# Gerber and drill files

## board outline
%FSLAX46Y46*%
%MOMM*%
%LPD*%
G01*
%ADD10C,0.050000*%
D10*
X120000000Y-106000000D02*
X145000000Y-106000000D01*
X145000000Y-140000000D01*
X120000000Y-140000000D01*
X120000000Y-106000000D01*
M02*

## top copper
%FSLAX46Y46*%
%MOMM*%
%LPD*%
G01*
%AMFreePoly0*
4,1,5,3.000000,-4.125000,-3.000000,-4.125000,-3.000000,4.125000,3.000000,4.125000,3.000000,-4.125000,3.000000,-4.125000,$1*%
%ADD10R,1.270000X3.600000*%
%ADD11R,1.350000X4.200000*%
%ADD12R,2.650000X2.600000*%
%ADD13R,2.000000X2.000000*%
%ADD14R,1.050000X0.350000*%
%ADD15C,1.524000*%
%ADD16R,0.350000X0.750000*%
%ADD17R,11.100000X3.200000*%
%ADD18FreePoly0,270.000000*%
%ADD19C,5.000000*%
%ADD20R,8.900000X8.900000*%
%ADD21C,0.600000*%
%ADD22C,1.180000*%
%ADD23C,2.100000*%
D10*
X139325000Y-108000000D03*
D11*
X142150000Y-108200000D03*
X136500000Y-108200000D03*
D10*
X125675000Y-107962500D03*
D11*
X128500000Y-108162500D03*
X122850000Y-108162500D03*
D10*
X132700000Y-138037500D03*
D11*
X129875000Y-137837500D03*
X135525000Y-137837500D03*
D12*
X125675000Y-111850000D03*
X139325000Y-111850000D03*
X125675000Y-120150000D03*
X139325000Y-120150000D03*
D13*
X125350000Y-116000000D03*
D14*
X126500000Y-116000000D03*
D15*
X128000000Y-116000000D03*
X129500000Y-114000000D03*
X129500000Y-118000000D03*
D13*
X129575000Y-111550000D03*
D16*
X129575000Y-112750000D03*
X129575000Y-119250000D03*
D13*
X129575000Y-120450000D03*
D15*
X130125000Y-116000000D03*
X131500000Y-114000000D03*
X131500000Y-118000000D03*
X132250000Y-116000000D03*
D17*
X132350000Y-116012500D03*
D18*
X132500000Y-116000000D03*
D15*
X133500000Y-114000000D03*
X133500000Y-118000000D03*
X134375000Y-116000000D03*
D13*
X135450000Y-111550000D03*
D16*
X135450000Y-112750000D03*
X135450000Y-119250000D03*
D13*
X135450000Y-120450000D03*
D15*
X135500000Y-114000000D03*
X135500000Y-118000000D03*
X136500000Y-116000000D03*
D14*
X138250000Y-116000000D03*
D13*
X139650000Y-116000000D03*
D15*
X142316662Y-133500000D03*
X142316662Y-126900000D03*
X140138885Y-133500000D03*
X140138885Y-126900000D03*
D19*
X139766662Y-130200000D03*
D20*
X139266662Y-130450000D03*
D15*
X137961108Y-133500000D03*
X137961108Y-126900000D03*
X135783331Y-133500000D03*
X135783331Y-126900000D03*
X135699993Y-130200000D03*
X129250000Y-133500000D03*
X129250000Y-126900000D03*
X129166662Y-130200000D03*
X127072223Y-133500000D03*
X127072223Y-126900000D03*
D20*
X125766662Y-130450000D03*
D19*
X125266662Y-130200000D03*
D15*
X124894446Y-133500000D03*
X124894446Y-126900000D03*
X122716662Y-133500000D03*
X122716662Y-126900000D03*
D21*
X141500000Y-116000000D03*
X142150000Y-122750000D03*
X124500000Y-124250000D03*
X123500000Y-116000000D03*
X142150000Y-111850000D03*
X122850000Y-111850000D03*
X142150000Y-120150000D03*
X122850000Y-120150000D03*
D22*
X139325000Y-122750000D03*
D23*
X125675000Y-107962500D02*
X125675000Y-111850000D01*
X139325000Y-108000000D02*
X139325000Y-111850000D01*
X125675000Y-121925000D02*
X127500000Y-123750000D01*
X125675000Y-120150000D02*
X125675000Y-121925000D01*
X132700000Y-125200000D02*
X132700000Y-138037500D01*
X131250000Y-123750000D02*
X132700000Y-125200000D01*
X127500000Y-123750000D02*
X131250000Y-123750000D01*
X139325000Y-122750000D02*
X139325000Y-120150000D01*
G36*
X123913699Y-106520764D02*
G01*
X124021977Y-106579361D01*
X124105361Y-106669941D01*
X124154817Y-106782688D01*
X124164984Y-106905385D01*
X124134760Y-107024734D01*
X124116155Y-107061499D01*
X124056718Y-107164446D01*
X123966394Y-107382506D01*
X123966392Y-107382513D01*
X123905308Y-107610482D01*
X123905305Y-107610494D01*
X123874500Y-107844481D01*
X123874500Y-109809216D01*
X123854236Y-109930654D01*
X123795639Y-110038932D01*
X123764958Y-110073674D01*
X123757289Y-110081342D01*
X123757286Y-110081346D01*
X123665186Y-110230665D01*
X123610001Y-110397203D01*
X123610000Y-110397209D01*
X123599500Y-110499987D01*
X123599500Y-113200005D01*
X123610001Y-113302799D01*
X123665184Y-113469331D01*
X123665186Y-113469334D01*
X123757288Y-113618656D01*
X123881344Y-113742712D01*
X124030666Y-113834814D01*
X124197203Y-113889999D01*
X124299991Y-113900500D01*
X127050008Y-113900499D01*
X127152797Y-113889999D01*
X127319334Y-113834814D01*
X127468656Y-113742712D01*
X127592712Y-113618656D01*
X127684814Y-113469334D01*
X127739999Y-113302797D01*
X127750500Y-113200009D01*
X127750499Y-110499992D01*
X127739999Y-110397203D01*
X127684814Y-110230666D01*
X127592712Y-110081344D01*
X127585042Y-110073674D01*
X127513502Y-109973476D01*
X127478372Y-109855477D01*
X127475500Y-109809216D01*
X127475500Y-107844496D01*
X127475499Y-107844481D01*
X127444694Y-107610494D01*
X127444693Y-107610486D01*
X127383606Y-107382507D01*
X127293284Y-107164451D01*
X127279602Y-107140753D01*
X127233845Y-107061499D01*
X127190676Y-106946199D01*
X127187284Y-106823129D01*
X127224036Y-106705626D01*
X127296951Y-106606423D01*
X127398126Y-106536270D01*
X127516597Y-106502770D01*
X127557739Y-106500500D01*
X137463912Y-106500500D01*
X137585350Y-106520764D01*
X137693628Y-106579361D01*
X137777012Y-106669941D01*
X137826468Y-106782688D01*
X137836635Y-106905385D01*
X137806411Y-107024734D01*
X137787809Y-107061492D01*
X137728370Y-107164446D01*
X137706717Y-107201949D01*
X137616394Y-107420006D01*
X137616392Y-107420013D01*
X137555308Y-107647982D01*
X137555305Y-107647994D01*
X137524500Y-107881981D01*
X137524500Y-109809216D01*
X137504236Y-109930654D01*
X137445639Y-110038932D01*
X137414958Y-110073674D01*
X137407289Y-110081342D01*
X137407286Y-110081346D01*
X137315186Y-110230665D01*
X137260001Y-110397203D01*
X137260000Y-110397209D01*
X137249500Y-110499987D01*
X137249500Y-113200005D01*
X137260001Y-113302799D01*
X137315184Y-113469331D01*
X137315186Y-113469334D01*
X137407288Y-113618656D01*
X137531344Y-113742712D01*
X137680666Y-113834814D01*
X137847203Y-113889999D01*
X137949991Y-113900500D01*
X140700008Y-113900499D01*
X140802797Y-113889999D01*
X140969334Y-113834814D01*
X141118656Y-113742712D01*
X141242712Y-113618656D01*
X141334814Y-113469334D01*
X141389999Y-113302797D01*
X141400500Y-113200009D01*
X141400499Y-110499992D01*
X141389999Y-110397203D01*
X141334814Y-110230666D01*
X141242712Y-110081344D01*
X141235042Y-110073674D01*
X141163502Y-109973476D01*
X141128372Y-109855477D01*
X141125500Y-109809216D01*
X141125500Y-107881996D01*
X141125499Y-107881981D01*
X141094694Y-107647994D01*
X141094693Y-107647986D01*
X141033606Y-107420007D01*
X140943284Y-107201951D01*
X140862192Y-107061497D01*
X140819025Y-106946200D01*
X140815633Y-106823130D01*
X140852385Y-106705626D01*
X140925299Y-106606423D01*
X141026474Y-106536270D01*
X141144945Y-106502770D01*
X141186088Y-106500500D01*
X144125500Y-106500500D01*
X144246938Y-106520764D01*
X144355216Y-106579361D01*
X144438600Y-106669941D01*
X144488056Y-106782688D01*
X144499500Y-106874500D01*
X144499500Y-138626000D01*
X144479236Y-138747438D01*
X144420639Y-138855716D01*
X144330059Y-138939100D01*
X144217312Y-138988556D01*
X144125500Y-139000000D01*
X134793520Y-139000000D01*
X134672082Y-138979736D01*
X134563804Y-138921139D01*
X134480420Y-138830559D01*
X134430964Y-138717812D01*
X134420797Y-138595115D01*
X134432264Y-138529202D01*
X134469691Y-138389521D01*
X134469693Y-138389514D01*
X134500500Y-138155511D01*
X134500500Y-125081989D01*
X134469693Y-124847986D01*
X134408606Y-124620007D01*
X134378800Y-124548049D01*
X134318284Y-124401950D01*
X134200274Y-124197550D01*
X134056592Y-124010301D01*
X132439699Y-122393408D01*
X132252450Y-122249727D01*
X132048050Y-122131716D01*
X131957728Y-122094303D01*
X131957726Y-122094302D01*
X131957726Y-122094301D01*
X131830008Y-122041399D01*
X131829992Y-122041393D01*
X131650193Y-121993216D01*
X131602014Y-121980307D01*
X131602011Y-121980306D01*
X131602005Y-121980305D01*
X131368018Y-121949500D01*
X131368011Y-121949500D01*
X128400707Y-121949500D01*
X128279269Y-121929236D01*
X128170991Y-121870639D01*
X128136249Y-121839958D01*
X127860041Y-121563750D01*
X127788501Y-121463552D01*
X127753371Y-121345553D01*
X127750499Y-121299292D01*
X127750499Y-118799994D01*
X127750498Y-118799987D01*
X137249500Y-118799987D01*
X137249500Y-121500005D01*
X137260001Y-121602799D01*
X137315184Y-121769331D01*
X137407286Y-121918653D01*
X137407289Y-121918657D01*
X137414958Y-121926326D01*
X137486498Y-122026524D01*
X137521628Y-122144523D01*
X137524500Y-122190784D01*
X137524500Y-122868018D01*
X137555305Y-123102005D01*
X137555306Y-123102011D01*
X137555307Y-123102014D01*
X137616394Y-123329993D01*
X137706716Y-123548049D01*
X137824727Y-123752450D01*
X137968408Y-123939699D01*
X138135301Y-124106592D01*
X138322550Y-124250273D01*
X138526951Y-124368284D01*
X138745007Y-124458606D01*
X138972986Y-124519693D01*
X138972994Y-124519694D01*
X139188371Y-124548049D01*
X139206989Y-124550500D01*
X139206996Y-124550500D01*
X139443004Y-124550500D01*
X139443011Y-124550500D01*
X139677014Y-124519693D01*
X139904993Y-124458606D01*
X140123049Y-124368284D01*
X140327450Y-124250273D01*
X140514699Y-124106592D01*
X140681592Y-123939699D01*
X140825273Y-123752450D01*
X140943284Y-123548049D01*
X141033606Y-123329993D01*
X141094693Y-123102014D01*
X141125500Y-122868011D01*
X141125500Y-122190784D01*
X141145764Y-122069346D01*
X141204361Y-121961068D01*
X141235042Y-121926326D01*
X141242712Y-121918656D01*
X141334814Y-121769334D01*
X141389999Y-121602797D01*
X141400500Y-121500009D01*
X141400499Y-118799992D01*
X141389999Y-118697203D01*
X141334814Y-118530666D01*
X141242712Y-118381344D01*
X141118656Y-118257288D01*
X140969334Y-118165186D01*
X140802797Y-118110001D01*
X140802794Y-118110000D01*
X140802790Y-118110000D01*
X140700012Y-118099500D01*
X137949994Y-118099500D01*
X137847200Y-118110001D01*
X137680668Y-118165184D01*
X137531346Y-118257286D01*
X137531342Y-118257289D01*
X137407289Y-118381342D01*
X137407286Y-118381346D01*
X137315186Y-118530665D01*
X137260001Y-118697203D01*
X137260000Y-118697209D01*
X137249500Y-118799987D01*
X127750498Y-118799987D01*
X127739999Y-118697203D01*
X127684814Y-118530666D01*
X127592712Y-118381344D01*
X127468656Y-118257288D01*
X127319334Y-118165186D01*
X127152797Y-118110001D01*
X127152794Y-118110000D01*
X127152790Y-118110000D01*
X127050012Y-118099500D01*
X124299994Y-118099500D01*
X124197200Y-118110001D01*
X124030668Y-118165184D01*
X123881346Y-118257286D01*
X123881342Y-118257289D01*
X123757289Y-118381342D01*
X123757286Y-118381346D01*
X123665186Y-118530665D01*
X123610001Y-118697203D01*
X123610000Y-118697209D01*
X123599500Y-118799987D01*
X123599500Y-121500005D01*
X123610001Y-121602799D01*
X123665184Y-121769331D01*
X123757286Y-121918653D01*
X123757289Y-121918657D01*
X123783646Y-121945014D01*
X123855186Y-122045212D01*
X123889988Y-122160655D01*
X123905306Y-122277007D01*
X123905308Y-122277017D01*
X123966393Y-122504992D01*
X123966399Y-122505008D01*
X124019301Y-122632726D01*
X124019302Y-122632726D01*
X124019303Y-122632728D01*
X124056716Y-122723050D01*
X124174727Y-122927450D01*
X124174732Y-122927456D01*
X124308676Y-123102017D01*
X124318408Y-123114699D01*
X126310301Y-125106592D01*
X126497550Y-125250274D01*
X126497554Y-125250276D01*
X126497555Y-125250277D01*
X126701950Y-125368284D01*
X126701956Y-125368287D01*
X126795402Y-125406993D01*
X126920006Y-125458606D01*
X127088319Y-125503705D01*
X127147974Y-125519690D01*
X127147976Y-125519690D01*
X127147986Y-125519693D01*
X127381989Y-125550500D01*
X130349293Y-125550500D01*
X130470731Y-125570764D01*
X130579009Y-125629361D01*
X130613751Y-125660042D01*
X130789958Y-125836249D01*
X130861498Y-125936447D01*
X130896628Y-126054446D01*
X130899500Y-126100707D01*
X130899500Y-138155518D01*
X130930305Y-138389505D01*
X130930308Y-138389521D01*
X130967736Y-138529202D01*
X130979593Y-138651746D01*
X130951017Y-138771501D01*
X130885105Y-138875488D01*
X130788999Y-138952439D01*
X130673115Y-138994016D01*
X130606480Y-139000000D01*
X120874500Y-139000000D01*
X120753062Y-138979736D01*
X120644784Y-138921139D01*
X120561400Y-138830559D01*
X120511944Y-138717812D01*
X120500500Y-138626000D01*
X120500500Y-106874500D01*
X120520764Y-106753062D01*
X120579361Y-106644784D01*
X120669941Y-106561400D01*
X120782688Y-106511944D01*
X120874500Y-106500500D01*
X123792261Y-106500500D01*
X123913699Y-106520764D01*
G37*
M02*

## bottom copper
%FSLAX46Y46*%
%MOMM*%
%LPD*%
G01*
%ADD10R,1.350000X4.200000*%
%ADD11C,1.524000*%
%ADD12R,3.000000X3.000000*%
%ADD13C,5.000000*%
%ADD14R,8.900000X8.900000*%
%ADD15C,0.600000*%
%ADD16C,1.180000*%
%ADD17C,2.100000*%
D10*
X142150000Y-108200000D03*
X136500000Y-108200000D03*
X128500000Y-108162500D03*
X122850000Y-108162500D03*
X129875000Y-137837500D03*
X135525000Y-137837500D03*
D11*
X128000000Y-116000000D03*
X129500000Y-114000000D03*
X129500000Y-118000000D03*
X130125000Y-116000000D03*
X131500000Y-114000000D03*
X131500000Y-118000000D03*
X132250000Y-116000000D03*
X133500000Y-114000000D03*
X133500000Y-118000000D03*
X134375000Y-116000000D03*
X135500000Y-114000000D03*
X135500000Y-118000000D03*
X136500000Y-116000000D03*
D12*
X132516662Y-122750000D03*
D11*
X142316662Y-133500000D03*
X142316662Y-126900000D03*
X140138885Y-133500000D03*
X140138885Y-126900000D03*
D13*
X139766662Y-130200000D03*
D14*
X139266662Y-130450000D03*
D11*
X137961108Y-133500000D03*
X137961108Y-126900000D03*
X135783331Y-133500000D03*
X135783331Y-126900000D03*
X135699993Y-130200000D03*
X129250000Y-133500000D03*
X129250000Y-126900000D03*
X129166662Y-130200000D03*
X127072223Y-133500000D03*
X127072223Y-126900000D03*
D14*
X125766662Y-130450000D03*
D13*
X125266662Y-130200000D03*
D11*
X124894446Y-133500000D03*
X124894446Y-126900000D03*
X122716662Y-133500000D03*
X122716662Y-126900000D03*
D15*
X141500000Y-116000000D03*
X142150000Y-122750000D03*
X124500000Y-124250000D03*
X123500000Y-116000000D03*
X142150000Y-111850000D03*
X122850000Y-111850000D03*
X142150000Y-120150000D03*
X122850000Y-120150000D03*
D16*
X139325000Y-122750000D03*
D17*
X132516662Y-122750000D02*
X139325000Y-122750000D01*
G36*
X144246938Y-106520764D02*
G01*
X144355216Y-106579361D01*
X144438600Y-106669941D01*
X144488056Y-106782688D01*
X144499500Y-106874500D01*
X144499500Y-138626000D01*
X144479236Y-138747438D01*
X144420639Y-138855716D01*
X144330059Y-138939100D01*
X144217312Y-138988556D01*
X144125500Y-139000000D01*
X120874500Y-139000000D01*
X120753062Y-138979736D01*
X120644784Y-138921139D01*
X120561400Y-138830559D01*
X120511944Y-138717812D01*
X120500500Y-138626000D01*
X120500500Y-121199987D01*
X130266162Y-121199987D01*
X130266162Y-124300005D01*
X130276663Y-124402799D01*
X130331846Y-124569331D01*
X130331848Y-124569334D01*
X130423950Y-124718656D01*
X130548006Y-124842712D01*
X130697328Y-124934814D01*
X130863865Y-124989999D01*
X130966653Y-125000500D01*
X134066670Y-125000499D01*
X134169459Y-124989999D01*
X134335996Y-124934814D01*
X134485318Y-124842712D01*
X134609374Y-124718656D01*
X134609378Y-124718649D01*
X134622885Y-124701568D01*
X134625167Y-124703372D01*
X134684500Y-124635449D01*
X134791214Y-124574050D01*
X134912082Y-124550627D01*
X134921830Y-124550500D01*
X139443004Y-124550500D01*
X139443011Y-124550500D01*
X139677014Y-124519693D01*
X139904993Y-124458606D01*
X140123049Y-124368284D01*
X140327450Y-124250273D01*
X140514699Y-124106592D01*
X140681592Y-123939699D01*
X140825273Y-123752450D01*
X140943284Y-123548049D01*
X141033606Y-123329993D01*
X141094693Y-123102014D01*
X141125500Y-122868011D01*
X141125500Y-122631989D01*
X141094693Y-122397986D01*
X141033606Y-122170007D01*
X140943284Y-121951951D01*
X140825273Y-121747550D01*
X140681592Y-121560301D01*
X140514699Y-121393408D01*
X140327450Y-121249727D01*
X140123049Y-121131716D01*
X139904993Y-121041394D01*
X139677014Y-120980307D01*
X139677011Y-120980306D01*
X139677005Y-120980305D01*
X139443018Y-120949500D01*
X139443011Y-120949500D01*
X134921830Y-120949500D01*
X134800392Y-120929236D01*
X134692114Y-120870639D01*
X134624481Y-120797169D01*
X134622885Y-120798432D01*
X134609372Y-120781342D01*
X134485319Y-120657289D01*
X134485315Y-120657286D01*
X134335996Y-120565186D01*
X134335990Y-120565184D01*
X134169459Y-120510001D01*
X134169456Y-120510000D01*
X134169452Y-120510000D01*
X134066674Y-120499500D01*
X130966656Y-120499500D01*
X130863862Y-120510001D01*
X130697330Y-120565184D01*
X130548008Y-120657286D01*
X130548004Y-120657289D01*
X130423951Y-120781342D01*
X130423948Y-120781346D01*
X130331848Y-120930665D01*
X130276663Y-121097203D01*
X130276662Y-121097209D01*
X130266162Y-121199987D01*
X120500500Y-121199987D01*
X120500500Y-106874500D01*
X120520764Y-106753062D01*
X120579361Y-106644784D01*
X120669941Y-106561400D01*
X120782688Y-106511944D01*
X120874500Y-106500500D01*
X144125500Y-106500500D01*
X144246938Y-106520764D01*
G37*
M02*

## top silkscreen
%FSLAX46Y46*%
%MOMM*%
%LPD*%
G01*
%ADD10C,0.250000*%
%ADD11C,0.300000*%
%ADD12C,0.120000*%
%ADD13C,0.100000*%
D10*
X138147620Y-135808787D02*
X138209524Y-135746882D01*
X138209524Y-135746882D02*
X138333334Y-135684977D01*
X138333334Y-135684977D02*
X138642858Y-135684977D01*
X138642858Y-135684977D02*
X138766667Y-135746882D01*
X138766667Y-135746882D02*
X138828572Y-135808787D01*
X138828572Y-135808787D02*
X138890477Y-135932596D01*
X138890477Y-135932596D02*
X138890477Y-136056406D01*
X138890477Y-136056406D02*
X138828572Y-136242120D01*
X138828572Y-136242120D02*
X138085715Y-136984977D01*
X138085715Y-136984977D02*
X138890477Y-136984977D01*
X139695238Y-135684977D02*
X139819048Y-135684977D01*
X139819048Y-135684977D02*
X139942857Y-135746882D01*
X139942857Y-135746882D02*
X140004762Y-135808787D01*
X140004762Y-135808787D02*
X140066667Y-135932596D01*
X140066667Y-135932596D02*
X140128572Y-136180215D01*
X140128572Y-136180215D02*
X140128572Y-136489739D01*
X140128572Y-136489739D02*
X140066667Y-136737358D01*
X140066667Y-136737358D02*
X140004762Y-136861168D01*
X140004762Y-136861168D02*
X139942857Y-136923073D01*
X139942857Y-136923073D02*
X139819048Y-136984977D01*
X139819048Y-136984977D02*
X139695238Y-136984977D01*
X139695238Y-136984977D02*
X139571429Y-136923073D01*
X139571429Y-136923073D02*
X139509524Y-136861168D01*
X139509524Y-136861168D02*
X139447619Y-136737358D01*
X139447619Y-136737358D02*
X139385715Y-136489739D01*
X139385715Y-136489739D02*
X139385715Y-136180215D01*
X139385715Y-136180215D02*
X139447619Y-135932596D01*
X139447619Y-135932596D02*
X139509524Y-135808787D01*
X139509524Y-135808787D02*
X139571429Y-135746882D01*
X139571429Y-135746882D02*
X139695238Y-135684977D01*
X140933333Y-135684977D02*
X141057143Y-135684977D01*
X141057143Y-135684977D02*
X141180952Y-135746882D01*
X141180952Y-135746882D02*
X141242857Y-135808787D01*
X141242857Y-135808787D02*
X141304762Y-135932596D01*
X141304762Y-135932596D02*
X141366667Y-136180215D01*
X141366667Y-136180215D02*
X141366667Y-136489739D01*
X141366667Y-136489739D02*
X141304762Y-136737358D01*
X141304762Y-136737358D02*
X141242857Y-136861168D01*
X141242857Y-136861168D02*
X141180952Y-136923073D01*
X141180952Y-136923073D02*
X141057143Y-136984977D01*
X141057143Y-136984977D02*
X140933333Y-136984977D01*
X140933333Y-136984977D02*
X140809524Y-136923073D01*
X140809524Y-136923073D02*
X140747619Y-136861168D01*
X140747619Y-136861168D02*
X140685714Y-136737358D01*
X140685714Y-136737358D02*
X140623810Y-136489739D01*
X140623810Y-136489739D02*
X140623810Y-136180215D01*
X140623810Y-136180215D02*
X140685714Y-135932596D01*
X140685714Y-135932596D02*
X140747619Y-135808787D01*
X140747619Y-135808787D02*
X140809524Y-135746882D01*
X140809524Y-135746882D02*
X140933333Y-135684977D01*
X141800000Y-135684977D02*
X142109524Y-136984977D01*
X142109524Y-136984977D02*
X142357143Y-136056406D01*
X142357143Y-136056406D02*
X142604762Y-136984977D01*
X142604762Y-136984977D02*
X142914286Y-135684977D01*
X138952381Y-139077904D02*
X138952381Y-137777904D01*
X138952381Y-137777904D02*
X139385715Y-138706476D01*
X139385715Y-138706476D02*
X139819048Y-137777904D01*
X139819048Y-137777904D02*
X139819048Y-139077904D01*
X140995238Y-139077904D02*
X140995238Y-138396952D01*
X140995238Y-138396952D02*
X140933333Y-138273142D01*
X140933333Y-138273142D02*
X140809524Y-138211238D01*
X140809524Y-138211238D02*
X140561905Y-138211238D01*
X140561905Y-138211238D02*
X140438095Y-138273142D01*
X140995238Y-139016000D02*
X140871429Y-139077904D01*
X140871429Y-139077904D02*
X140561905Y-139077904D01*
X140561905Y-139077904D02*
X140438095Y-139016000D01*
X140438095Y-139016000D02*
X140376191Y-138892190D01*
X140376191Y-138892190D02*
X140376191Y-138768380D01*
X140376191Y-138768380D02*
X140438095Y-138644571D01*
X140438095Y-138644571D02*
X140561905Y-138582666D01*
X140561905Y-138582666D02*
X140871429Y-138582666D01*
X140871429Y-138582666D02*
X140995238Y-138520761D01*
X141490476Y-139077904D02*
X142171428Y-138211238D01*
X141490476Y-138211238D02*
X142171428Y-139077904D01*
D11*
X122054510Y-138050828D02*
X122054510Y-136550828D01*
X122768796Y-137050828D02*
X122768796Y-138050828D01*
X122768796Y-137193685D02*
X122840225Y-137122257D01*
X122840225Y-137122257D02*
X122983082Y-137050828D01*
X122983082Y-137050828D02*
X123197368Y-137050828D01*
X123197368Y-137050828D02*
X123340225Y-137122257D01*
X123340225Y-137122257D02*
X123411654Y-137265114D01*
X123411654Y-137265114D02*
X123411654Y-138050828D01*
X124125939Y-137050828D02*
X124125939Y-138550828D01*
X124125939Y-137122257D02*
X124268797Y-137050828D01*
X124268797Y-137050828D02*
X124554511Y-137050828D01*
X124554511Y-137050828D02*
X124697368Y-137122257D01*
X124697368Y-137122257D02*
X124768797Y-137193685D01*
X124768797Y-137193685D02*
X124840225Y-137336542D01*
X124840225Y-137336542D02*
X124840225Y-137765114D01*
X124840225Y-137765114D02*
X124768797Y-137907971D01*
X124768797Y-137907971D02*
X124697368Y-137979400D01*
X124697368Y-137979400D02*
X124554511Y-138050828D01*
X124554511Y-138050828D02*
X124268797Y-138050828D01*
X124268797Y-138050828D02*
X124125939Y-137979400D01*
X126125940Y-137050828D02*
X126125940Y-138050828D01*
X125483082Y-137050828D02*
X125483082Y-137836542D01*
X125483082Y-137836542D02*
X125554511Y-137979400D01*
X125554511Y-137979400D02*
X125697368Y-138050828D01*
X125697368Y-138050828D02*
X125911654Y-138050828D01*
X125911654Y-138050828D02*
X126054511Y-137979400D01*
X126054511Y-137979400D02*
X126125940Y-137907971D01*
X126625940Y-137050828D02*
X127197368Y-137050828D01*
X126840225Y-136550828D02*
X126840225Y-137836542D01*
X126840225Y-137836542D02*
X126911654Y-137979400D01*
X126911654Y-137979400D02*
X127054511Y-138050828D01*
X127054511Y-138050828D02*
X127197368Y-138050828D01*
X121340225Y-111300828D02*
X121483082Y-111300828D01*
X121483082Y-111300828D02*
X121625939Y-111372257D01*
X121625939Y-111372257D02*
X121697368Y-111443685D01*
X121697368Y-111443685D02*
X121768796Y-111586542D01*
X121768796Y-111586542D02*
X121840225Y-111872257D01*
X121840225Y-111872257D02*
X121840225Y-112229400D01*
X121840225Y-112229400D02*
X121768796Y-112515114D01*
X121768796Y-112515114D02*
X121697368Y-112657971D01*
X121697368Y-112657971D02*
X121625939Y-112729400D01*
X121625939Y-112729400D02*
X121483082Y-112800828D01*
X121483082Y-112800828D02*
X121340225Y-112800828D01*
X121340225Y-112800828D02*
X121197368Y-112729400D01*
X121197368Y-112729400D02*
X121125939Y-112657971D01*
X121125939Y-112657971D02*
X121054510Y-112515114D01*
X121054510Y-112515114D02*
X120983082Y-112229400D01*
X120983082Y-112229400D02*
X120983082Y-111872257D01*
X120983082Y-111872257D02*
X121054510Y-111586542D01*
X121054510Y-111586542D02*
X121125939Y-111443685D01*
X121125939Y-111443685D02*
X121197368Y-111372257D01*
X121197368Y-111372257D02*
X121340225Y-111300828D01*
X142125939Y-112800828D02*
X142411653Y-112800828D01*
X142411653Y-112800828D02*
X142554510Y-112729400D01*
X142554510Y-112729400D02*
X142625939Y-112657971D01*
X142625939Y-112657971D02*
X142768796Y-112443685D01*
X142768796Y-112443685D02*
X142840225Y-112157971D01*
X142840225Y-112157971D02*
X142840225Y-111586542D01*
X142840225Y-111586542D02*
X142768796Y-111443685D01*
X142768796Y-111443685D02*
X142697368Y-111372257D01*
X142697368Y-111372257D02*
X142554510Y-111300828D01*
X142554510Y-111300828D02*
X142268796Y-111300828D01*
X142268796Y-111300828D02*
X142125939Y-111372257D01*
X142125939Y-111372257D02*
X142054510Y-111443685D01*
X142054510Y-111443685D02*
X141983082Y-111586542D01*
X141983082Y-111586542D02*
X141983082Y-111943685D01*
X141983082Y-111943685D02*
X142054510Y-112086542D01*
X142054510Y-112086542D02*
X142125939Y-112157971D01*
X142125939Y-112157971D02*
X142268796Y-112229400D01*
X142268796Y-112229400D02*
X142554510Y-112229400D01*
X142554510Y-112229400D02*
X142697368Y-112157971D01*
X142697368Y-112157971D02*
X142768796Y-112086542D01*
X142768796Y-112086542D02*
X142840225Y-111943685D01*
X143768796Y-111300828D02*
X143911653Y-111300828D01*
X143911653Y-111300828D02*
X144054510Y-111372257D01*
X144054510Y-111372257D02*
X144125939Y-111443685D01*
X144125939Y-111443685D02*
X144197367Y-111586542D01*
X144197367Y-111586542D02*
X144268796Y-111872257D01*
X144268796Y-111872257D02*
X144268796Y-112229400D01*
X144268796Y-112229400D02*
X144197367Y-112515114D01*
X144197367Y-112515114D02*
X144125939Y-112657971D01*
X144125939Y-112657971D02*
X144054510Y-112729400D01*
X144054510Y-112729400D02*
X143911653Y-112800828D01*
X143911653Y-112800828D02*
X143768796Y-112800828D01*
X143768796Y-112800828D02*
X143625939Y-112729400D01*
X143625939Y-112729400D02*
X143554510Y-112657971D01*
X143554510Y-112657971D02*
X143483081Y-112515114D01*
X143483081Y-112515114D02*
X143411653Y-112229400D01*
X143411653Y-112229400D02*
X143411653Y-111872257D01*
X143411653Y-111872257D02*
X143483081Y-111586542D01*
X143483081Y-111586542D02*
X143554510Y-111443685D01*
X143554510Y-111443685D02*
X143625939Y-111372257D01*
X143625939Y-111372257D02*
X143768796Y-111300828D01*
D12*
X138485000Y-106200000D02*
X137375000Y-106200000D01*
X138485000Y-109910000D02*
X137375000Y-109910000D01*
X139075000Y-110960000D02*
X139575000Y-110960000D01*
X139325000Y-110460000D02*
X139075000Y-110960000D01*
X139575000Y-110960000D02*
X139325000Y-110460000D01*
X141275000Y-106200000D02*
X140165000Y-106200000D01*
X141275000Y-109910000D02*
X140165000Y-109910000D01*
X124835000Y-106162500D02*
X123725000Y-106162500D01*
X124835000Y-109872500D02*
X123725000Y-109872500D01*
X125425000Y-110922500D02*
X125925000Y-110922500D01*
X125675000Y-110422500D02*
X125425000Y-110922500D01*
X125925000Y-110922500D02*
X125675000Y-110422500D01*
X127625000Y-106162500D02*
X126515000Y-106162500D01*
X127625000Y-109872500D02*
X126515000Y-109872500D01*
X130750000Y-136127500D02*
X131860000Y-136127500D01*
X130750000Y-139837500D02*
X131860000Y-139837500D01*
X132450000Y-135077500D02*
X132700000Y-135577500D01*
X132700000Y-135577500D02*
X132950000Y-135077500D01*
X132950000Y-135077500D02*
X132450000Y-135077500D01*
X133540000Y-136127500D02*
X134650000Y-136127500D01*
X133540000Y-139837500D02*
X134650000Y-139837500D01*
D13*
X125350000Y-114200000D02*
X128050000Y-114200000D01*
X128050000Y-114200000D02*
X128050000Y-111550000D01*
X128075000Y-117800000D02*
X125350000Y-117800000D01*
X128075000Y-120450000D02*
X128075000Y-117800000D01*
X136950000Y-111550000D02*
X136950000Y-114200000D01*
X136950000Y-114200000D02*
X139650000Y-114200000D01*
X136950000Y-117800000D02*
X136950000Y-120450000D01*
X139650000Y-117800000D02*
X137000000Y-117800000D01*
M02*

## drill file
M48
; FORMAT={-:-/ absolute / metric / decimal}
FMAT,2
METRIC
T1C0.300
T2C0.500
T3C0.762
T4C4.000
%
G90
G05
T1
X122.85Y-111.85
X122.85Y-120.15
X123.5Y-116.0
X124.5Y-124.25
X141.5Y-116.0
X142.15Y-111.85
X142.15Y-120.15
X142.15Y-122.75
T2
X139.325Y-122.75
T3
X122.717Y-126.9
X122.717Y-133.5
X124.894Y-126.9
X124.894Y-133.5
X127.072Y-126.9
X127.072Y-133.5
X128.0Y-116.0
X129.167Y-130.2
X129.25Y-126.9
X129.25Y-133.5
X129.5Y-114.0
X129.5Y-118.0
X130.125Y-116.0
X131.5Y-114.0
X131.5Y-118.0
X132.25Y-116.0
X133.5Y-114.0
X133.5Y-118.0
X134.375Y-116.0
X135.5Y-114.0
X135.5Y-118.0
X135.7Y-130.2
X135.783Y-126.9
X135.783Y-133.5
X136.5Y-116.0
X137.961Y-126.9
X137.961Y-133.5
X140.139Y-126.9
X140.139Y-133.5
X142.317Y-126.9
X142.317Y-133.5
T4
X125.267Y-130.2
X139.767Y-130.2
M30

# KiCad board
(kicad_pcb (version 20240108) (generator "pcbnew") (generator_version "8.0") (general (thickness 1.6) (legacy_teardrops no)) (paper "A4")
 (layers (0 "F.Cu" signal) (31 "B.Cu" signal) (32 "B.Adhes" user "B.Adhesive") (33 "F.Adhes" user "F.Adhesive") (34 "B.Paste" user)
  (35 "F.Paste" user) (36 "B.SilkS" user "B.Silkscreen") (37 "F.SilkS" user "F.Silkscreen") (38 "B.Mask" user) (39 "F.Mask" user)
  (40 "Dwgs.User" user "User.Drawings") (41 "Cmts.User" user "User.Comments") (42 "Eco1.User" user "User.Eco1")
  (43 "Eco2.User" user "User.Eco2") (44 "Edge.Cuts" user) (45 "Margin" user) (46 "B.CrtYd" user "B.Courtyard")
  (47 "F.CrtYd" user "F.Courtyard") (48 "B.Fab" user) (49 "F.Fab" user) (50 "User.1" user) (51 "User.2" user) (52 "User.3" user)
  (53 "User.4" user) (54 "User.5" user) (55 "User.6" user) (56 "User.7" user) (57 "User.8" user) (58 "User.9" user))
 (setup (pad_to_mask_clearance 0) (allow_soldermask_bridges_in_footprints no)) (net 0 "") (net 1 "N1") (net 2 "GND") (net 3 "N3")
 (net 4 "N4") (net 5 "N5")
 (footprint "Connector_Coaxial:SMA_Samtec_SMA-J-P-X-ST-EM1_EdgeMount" (layer "F.Cu") (at 139.325 108.2 180)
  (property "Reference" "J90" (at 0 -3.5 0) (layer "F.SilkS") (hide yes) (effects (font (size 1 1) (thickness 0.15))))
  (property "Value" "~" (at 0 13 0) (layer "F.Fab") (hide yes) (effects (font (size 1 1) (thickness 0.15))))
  (fp_line (start 0.84 2) (end 1.95 2) (stroke (width 0.12) (type solid)) (layer "F.SilkS"))
  (fp_line (start 0.84 -1.71) (end 1.95 -1.71) (stroke (width 0.12) (type solid)) (layer "F.SilkS"))
  (fp_line (start 0.25 -2.76) (end -0.25 -2.76) (stroke (width 0.12) (type solid)) (layer "F.SilkS"))
  (fp_line (start 0 -2.26) (end 0.25 -2.76) (stroke (width 0.12) (type solid)) (layer "F.SilkS"))
  (fp_line (start -0.25 -2.76) (end 0 -2.26) (stroke (width 0.12) (type solid)) (layer "F.SilkS"))
  (fp_line (start -1.95 2) (end -0.84 2) (stroke (width 0.12) (type solid)) (layer "F.SilkS"))
  (fp_line (start -1.95 -1.71) (end -0.84 -1.71) (stroke (width 0.12) (type solid)) (layer "F.SilkS"))
  (pad "1" smd rect (at 0 0.2 180) (size 1.27 3.6) (layers "F.Cu" "F.Paste" "F.Mask") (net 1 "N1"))
  (pad "2" smd rect (at -2.825 0 180) (size 1.35 4.2) (layers "F.Cu" "F.Paste" "F.Mask") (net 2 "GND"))
  (pad "2" smd rect (at -2.825 0 180) (size 1.35 4.2) (layers "B.Cu" "B.Paste" "B.Mask") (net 2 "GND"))
  (pad "2" smd rect (at 2.825 0 180) (size 1.35 4.2) (layers "F.Cu" "F.Paste" "F.Mask") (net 2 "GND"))
  (pad "2" smd rect (at 2.825 0 180) (size 1.35 4.2) (layers "B.Cu" "B.Paste" "B.Mask") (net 2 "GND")))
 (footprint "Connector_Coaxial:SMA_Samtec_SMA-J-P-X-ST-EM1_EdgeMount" (layer "F.Cu") (at 125.675 108.1625 180)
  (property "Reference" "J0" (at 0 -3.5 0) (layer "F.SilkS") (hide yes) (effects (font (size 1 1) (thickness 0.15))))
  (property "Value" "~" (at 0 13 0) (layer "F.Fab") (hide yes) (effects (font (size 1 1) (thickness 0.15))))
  (fp_line (start 0.84 2) (end 1.95 2) (stroke (width 0.12) (type solid)) (layer "F.SilkS"))
  (fp_line (start 0.84 -1.71) (end 1.95 -1.71) (stroke (width 0.12) (type solid)) (layer "F.SilkS"))
  (fp_line (start 0.25 -2.76) (end -0.25 -2.76) (stroke (width 0.12) (type solid)) (layer "F.SilkS"))
  (fp_line (start 0 -2.26) (end 0.25 -2.76) (stroke (width 0.12) (type solid)) (layer "F.SilkS"))
  (fp_line (start -0.25 -2.76) (end 0 -2.26) (stroke (width 0.12) (type solid)) (layer "F.SilkS"))
  (fp_line (start -1.95 2) (end -0.84 2) (stroke (width 0.12) (type solid)) (layer "F.SilkS"))
  (fp_line (start -1.95 -1.71) (end -0.84 -1.71) (stroke (width 0.12) (type solid)) (layer "F.SilkS"))
  (pad "1" smd rect (at 0 0.2 180) (size 1.27 3.6) (layers "F.Cu" "F.Paste" "F.Mask") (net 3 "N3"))
  (pad "2" smd rect (at -2.825 0 180) (size 1.35 4.2) (layers "F.Cu" "F.Paste" "F.Mask") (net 2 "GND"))
  (pad "2" smd rect (at -2.825 0 180) (size 1.35 4.2) (layers "B.Cu" "B.Paste" "B.Mask") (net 2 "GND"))
  (pad "2" smd rect (at 2.825 0 180) (size 1.35 4.2) (layers "F.Cu" "F.Paste" "F.Mask") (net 2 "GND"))
  (pad "2" smd rect (at 2.825 0 180) (size 1.35 4.2) (layers "B.Cu" "B.Paste" "B.Mask") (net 2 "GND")))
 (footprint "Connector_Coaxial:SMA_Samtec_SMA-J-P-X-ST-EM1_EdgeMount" (layer "F.Cu") (at 132.7 137.8375)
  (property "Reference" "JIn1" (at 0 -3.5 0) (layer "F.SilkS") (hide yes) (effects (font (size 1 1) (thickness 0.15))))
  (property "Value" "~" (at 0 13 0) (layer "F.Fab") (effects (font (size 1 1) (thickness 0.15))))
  (fp_line (start -1.95 -1.71) (end -0.84 -1.71) (stroke (width 0.12) (type solid)) (layer "F.SilkS"))
  (fp_line (start -1.95 2) (end -0.84 2) (stroke (width 0.12) (type solid)) (layer "F.SilkS"))
  (fp_line (start -0.25 -2.76) (end 0 -2.26) (stroke (width 0.12) (type solid)) (layer "F.SilkS"))
  (fp_line (start 0 -2.26) (end 0.25 -2.76) (stroke (width 0.12) (type solid)) (layer "F.SilkS"))
  (fp_line (start 0.25 -2.76) (end -0.25 -2.76) (stroke (width 0.12) (type solid)) (layer "F.SilkS"))
  (fp_line (start 0.84 -1.71) (end 1.95 -1.71) (stroke (width 0.12) (type solid)) (layer "F.SilkS"))
  (fp_line (start 0.84 2) (end 1.95 2) (stroke (width 0.12) (type solid)) (layer "F.SilkS"))
  (pad "1" smd rect (at 0 0.2) (size 1.27 3.6) (layers "F.Cu" "F.Paste" "F.Mask") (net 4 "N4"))
  (pad "2" smd rect (at -2.825 0) (size 1.35 4.2) (layers "F.Cu" "F.Paste" "F.Mask") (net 2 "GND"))
  (pad "2" smd rect (at -2.825 0) (size 1.35 4.2) (layers "B.Cu" "B.Paste" "B.Mask") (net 2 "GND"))
  (pad "2" smd rect (at 2.825 0) (size 1.35 4.2) (layers "F.Cu" "F.Paste" "F.Mask") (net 2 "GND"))
  (pad "2" smd rect (at 2.825 0) (size 1.35 4.2) (layers "B.Cu" "B.Paste" "B.Mask") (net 2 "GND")))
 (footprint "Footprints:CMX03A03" (layer "F.Cu") (at 132.5 116)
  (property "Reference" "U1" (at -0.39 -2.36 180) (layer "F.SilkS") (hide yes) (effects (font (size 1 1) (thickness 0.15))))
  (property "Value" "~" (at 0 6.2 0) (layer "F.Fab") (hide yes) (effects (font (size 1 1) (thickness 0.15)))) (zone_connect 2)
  (fp_line (start -7.15 -1.8) (end -4.45 -1.8) (stroke (width 0.1) (type default)) (layer "F.SilkS"))
  (fp_line (start -4.45 -1.8) (end -4.45 -4.45) (stroke (width 0.1) (type default)) (layer "F.SilkS"))
  (fp_line (start -4.425 1.8) (end -7.15 1.8) (stroke (width 0.1) (type default)) (layer "F.SilkS"))
  (fp_line (start -4.425 4.45) (end -4.425 1.8) (stroke (width 0.1) (type default)) (layer "F.SilkS"))
  (fp_line (start 4.45 -4.45) (end 4.45 -1.8) (stroke (width 0.1) (type default)) (layer "F.SilkS"))
  (fp_line (start 4.45 -1.8) (end 7.15 -1.8) (stroke (width 0.1) (type default)) (layer "F.SilkS"))
  (fp_line (start 4.45 1.8) (end 4.45 4.45) (stroke (width 0.1) (type default)) (layer "F.SilkS"))
  (fp_line (start 7.15 1.8) (end 4.5 1.8) (stroke (width 0.1) (type default)) (layer "F.SilkS"))
  (pad "1" smd rect (at -6.825 -4.15 270) (size 2.6 2.65) (layers "F.Cu" "F.Paste" "F.Mask") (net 3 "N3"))
  (pad "2" smd rect (at 6.825 -4.15 270) (size 2.6 2.65) (layers "F.Cu" "F.Paste" "F.Mask") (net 1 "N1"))
  (pad "3" smd rect (at -6.825 4.15 270) (size 2.6 2.65) (layers "F.Cu" "F.Paste" "F.Mask") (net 4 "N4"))
  (pad "4" smd rect (at 6.825 4.15 270) (size 2.6 2.65) (layers "F.Cu" "F.Paste" "F.Mask") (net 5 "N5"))
  (pad "5" smd rect (at -7.15 0) (size 2 2) (layers "F.Cu" "F.Paste" "F.Mask") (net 2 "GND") (zone_connect 2))
  (pad "5" smd rect (at -6 0) (size 1.05 0.35) (layers "F.Cu" "F.Mask") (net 2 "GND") (zone_connect 2))
  (pad "5" thru_hole circle (at -4.5 0) (size 1.524 1.524) (drill 0.762) (layers "*.Cu" "*.Mask") (remove_unused_layers no) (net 2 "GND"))
  (pad "5" thru_hole circle (at -3 -2) (size 1.524 1.524) (drill 0.762) (layers "*.Cu" "*.Mask") (remove_unused_layers no) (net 2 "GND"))
  (pad "5" thru_hole circle (at -3 2) (size 1.524 1.524) (drill 0.762) (layers "*.Cu" "*.Mask") (remove_unused_layers no) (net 2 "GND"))
  (pad "5" smd rect (at -2.925 -4.45 270) (size 2 2) (layers "F.Cu" "F.Paste" "F.Mask") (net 2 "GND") (zone_connect 2))
  (pad "5" smd rect (at -2.925 -3.25 90) (size 0.75 0.35) (layers "F.Cu" "F.Mask") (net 2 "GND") (zone_connect 2))
  (pad "5" smd rect (at -2.925 3.25 90) (size 0.75 0.35) (layers "F.Cu" "F.Mask") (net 2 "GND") (zone_connect 2))
  (pad "5" smd rect (at -2.925 4.45 270) (size 2 2) (layers "F.Cu" "F.Paste" "F.Mask") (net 2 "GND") (zone_connect 2))
  (pad "5" thru_hole circle (at -2.375 0) (size 1.524 1.524) (drill 0.762) (layers "*.Cu" "*.Mask") (remove_unused_layers no) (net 2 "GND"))
  (pad "5" thru_hole circle (at -1 -2) (size 1.524 1.524) (drill 0.762) (layers "*.Cu" "*.Mask") (remove_unused_layers no) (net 2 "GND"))
  (pad "5" thru_hole circle (at -1 2) (size 1.524 1.524) (drill 0.762) (layers "*.Cu" "*.Mask") (remove_unused_layers no) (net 2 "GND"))
  (pad "5" thru_hole circle (at -0.25 0) (size 1.524 1.524) (drill 0.762) (layers "*.Cu" "*.Mask") (remove_unused_layers no) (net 2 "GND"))
  (pad "5" smd rect (at -0.15 0.0125) (size 11.1 3.2) (layers "F.Cu" "F.Mask") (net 2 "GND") (zone_connect 2))
  (pad "5" smd custom (at 0 0 270) (size 6 8.25) (layers "F.Cu" "F.Mask") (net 2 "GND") (zone_connect 2)
   (options (clearance outline) (anchor rect)) (primitives))
  (pad "5" thru_hole circle (at 1 -2) (size 1.524 1.524) (drill 0.762) (layers "*.Cu" "*.Mask") (remove_unused_layers no) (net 2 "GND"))
  (pad "5" thru_hole circle (at 1 2) (size 1.524 1.524) (drill 0.762) (layers "*.Cu" "*.Mask") (remove_unused_layers no) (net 2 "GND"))
  (pad "5" thru_hole circle (at 1.875 0) (size 1.524 1.524) (drill 0.762) (layers "*.Cu" "*.Mask") (remove_unused_layers no) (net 2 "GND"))
  (pad "5" smd rect (at 2.95 -4.45 270) (size 2 2) (layers "F.Cu" "F.Paste" "F.Mask") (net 2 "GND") (zone_connect 2))
  (pad "5" smd rect (at 2.95 -3.25 90) (size 0.75 0.35) (layers "F.Cu" "F.Mask") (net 2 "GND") (zone_connect 2))
  (pad "5" smd rect (at 2.95 3.25 90) (size 0.75 0.35) (layers "F.Cu" "F.Mask") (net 2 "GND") (zone_connect 2))
  (pad "5" smd rect (at 2.95 4.45 270) (size 2 2) (layers "F.Cu" "F.Paste" "F.Mask") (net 2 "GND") (zone_connect 2))
  (pad "5" thru_hole circle (at 3 -2) (size 1.524 1.524) (drill 0.762) (layers "*.Cu" "*.Mask") (remove_unused_layers no) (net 2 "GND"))
  (pad "5" thru_hole circle (at 3 2) (size 1.524 1.524) (drill 0.762) (layers "*.Cu" "*.Mask") (remove_unused_layers no) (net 2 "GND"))
  (pad "5" thru_hole circle (at 4 0) (size 1.524 1.524) (drill 0.762) (layers "*.Cu" "*.Mask") (remove_unused_layers no) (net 2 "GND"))
  (pad "5" smd rect (at 5.75 0) (size 1.05 0.35) (layers "F.Cu" "F.Mask") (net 2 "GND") (zone_connect 2))
  (pad "5" smd rect (at 7.15 0) (size 2 2) (layers "F.Cu" "F.Paste" "F.Mask") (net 2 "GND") (zone_connect 2)))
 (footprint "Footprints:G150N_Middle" (layer "B.Cu") (at 132.516662 130.75 180)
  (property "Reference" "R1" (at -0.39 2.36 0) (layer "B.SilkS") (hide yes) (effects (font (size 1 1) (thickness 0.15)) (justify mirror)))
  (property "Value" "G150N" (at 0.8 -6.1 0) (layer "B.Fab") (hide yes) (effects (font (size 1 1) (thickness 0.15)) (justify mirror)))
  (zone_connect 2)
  (pad "1" smd rect (at 0 8 270) (size 3 3) (layers "B.Cu" "B.Paste" "B.Mask") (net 5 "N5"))
  (pad "2" thru_hole circle (at -9.8 -2.75 180) (size 1.524 1.524) (drill 0.762) (layers "*.Cu" "*.Mask") (remove_unused_layers no)
   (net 2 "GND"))
  (pad "2" thru_hole circle (at -9.8 3.85 180) (size 1.524 1.524) (drill 0.762) (layers "*.Cu" "*.Mask") (remove_unused_layers no)
   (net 2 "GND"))
  (pad "2" thru_hole circle (at -7.622223 -2.75 180) (size 1.524 1.524) (drill 0.762) (layers "*.Cu" "*.Mask") (remove_unused_layers no)
   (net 2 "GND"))
  (pad "2" thru_hole circle (at -7.622223 3.85 180) (size 1.524 1.524) (drill 0.762) (layers "*.Cu" "*.Mask") (remove_unused_layers no)
   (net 2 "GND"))
  (pad "2" thru_hole circle (at -7.25 0.55 270) (size 5 5) (drill 4) (layers "*.Cu" "*.Mask") (remove_unused_layers no) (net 2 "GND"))
  (pad "2" smd rect (at -6.75 0.3 270) (size 8.9 8.9) (layers "F.Cu" "F.Mask") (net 2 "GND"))
  (pad "2" smd rect (at -6.75 0.3 270) (size 8.9 8.9) (layers "B.Cu" "B.Mask") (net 2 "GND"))
  (pad "2" thru_hole circle (at -5.444446 -2.75 180) (size 1.524 1.524) (drill 0.762) (layers "*.Cu" "*.Mask") (remove_unused_layers no)
   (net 2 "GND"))
  (pad "2" thru_hole circle (at -5.444446 3.85 180) (size 1.524 1.524) (drill 0.762) (layers "*.Cu" "*.Mask") (remove_unused_layers no)
   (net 2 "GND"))
  (pad "2" thru_hole circle (at -3.266669 -2.75 180) (size 1.524 1.524) (drill 0.762) (layers "*.Cu" "*.Mask") (remove_unused_layers no)
   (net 2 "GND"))
  (pad "2" thru_hole circle (at -3.266669 3.85 180) (size 1.524 1.524) (drill 0.762) (layers "*.Cu" "*.Mask") (remove_unused_layers no)
   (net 2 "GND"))
  (pad "2" thru_hole circle (at -3.183331 0.55 180) (size 1.524 1.524) (drill 0.762) (layers "*.Cu" "*.Mask") (remove_unused_layers no)
   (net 2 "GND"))
  (pad "2" thru_hole circle (at 3.266662 -2.75 180) (size 1.524 1.524) (drill 0.762) (layers "*.Cu" "*.Mask") (remove_unused_layers no)
   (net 2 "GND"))
  (pad "2" thru_hole circle (at 3.266662 3.85 180) (size 1.524 1.524) (drill 0.762) (layers "*.Cu" "*.Mask") (remove_unused_layers no)
   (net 2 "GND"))
  (pad "2" thru_hole circle (at 3.35 0.55 180) (size 1.524 1.524) (drill 0.762) (layers "*.Cu" "*.Mask") (remove_unused_layers no)
   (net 2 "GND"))
  (pad "2" thru_hole circle (at 5.444439 -2.75 180) (size 1.524 1.524) (drill 0.762) (layers "*.Cu" "*.Mask") (remove_unused_layers no)
   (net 2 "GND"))
  (pad "2" thru_hole circle (at 5.444439 3.85 180) (size 1.524 1.524) (drill 0.762) (layers "*.Cu" "*.Mask") (remove_unused_layers no)
   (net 2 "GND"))
  (pad "2" smd rect (at 6.75 0.3 270) (size 8.9 8.9) (layers "F.Cu" "F.Mask") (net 2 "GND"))
  (pad "2" smd rect (at 6.75 0.3 270) (size 8.9 8.9) (layers "B.Cu" "B.Mask") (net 2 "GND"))
  (pad "2" thru_hole circle (at 7.25 0.55 270) (size 5 5) (drill 4) (layers "*.Cu" "*.Mask") (remove_unused_layers no) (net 2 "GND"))
  (pad "2" thru_hole circle (at 7.622216 -2.75 180) (size 1.524 1.524) (drill 0.762) (layers "*.Cu" "*.Mask") (remove_unused_layers no)
   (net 2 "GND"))
  (pad "2" thru_hole circle (at 7.622216 3.85 180) (size 1.524 1.524) (drill 0.762) (layers "*.Cu" "*.Mask") (remove_unused_layers no)
   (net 2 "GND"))
  (pad "2" thru_hole circle (at 9.8 -2.75 180) (size 1.524 1.524) (drill 0.762) (layers "*.Cu" "*.Mask") (remove_unused_layers no)
   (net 2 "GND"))
  (pad "2" thru_hole circle (at 9.8 3.85 180) (size 1.524 1.524) (drill 0.762) (layers "*.Cu" "*.Mask") (remove_unused_layers no)
   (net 2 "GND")))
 (gr_rect (start 120 106) (end 145 140) (stroke (width 0.05) (type default)) (fill none) (layer "Edge.Cuts"))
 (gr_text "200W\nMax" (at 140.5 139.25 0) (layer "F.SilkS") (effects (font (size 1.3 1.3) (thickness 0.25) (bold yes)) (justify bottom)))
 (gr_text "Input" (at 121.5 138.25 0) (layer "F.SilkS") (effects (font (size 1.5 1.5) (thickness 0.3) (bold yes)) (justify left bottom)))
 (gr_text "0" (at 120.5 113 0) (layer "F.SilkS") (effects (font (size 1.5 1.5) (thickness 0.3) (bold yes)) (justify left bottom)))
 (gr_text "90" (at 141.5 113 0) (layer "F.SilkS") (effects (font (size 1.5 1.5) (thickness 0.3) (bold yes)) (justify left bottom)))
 (via (at 141.5 116) (size 0.6) (drill 0.3) (layers "F.Cu" "B.Cu") (free yes) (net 2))
 (via (at 142.15 122.75) (size 0.6) (drill 0.3) (layers "F.Cu" "B.Cu") (free yes) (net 2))
 (via (at 124.5 124.25) (size 0.6) (drill 0.3) (layers "F.Cu" "B.Cu") (free yes) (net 2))
 (via (at 123.5 116) (size 0.6) (drill 0.3) (layers "F.Cu" "B.Cu") (free yes) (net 2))
 (via (at 142.15 111.85) (size 0.6) (drill 0.3) (layers "F.Cu" "B.Cu") (free yes) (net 2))
 (via (at 122.85 111.85) (size 0.6) (drill 0.3) (layers "F.Cu" "B.Cu") (free yes) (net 2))
 (via (at 142.15 120.15) (size 0.6) (drill 0.3) (layers "F.Cu" "B.Cu") (free yes) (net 2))
 (via (at 122.85 120.15) (size 0.6) (drill 0.3) (layers "F.Cu" "B.Cu") (free yes) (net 2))
 (segment (start 125.675 107.9625) (end 125.675 111.85) (width 2.1) (layer "F.Cu") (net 3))
 (segment (start 139.325 108) (end 139.325 111.85) (width 2.1) (layer "F.Cu") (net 1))
 (segment (start 125.675 121.925) (end 127.5 123.75) (width 2.1) (layer "F.Cu") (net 4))
 (segment (start 125.675 120.15) (end 125.675 121.925) (width 2.1) (layer "F.Cu") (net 4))
 (segment (start 132.7 125.2) (end 132.7 138.0375) (width 2.1) (layer "F.Cu") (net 4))
 (segment (start 131.25 123.75) (end 132.7 125.2) (width 2.1) (layer "F.Cu") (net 4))
 (segment (start 127.5 123.75) (end 131.25 123.75) (width 2.1) (layer "F.Cu") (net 4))
 (segment (start 139.325 122.75) (end 139.325 120.15) (width 2.1) (layer "F.Cu") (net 5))
 (via (at 139.325 122.75) (size 1.18) (drill 0.5) (layers "F.Cu" "B.Cu") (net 5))
 (segment (start 132.516662 122.75) (end 139.325 122.75) (width 2.1) (layer "B.Cu") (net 5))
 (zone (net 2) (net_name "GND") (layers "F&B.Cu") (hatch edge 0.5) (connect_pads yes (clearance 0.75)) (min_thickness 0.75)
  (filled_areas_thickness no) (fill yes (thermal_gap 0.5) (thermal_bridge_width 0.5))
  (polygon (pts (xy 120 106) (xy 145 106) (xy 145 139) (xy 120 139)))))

